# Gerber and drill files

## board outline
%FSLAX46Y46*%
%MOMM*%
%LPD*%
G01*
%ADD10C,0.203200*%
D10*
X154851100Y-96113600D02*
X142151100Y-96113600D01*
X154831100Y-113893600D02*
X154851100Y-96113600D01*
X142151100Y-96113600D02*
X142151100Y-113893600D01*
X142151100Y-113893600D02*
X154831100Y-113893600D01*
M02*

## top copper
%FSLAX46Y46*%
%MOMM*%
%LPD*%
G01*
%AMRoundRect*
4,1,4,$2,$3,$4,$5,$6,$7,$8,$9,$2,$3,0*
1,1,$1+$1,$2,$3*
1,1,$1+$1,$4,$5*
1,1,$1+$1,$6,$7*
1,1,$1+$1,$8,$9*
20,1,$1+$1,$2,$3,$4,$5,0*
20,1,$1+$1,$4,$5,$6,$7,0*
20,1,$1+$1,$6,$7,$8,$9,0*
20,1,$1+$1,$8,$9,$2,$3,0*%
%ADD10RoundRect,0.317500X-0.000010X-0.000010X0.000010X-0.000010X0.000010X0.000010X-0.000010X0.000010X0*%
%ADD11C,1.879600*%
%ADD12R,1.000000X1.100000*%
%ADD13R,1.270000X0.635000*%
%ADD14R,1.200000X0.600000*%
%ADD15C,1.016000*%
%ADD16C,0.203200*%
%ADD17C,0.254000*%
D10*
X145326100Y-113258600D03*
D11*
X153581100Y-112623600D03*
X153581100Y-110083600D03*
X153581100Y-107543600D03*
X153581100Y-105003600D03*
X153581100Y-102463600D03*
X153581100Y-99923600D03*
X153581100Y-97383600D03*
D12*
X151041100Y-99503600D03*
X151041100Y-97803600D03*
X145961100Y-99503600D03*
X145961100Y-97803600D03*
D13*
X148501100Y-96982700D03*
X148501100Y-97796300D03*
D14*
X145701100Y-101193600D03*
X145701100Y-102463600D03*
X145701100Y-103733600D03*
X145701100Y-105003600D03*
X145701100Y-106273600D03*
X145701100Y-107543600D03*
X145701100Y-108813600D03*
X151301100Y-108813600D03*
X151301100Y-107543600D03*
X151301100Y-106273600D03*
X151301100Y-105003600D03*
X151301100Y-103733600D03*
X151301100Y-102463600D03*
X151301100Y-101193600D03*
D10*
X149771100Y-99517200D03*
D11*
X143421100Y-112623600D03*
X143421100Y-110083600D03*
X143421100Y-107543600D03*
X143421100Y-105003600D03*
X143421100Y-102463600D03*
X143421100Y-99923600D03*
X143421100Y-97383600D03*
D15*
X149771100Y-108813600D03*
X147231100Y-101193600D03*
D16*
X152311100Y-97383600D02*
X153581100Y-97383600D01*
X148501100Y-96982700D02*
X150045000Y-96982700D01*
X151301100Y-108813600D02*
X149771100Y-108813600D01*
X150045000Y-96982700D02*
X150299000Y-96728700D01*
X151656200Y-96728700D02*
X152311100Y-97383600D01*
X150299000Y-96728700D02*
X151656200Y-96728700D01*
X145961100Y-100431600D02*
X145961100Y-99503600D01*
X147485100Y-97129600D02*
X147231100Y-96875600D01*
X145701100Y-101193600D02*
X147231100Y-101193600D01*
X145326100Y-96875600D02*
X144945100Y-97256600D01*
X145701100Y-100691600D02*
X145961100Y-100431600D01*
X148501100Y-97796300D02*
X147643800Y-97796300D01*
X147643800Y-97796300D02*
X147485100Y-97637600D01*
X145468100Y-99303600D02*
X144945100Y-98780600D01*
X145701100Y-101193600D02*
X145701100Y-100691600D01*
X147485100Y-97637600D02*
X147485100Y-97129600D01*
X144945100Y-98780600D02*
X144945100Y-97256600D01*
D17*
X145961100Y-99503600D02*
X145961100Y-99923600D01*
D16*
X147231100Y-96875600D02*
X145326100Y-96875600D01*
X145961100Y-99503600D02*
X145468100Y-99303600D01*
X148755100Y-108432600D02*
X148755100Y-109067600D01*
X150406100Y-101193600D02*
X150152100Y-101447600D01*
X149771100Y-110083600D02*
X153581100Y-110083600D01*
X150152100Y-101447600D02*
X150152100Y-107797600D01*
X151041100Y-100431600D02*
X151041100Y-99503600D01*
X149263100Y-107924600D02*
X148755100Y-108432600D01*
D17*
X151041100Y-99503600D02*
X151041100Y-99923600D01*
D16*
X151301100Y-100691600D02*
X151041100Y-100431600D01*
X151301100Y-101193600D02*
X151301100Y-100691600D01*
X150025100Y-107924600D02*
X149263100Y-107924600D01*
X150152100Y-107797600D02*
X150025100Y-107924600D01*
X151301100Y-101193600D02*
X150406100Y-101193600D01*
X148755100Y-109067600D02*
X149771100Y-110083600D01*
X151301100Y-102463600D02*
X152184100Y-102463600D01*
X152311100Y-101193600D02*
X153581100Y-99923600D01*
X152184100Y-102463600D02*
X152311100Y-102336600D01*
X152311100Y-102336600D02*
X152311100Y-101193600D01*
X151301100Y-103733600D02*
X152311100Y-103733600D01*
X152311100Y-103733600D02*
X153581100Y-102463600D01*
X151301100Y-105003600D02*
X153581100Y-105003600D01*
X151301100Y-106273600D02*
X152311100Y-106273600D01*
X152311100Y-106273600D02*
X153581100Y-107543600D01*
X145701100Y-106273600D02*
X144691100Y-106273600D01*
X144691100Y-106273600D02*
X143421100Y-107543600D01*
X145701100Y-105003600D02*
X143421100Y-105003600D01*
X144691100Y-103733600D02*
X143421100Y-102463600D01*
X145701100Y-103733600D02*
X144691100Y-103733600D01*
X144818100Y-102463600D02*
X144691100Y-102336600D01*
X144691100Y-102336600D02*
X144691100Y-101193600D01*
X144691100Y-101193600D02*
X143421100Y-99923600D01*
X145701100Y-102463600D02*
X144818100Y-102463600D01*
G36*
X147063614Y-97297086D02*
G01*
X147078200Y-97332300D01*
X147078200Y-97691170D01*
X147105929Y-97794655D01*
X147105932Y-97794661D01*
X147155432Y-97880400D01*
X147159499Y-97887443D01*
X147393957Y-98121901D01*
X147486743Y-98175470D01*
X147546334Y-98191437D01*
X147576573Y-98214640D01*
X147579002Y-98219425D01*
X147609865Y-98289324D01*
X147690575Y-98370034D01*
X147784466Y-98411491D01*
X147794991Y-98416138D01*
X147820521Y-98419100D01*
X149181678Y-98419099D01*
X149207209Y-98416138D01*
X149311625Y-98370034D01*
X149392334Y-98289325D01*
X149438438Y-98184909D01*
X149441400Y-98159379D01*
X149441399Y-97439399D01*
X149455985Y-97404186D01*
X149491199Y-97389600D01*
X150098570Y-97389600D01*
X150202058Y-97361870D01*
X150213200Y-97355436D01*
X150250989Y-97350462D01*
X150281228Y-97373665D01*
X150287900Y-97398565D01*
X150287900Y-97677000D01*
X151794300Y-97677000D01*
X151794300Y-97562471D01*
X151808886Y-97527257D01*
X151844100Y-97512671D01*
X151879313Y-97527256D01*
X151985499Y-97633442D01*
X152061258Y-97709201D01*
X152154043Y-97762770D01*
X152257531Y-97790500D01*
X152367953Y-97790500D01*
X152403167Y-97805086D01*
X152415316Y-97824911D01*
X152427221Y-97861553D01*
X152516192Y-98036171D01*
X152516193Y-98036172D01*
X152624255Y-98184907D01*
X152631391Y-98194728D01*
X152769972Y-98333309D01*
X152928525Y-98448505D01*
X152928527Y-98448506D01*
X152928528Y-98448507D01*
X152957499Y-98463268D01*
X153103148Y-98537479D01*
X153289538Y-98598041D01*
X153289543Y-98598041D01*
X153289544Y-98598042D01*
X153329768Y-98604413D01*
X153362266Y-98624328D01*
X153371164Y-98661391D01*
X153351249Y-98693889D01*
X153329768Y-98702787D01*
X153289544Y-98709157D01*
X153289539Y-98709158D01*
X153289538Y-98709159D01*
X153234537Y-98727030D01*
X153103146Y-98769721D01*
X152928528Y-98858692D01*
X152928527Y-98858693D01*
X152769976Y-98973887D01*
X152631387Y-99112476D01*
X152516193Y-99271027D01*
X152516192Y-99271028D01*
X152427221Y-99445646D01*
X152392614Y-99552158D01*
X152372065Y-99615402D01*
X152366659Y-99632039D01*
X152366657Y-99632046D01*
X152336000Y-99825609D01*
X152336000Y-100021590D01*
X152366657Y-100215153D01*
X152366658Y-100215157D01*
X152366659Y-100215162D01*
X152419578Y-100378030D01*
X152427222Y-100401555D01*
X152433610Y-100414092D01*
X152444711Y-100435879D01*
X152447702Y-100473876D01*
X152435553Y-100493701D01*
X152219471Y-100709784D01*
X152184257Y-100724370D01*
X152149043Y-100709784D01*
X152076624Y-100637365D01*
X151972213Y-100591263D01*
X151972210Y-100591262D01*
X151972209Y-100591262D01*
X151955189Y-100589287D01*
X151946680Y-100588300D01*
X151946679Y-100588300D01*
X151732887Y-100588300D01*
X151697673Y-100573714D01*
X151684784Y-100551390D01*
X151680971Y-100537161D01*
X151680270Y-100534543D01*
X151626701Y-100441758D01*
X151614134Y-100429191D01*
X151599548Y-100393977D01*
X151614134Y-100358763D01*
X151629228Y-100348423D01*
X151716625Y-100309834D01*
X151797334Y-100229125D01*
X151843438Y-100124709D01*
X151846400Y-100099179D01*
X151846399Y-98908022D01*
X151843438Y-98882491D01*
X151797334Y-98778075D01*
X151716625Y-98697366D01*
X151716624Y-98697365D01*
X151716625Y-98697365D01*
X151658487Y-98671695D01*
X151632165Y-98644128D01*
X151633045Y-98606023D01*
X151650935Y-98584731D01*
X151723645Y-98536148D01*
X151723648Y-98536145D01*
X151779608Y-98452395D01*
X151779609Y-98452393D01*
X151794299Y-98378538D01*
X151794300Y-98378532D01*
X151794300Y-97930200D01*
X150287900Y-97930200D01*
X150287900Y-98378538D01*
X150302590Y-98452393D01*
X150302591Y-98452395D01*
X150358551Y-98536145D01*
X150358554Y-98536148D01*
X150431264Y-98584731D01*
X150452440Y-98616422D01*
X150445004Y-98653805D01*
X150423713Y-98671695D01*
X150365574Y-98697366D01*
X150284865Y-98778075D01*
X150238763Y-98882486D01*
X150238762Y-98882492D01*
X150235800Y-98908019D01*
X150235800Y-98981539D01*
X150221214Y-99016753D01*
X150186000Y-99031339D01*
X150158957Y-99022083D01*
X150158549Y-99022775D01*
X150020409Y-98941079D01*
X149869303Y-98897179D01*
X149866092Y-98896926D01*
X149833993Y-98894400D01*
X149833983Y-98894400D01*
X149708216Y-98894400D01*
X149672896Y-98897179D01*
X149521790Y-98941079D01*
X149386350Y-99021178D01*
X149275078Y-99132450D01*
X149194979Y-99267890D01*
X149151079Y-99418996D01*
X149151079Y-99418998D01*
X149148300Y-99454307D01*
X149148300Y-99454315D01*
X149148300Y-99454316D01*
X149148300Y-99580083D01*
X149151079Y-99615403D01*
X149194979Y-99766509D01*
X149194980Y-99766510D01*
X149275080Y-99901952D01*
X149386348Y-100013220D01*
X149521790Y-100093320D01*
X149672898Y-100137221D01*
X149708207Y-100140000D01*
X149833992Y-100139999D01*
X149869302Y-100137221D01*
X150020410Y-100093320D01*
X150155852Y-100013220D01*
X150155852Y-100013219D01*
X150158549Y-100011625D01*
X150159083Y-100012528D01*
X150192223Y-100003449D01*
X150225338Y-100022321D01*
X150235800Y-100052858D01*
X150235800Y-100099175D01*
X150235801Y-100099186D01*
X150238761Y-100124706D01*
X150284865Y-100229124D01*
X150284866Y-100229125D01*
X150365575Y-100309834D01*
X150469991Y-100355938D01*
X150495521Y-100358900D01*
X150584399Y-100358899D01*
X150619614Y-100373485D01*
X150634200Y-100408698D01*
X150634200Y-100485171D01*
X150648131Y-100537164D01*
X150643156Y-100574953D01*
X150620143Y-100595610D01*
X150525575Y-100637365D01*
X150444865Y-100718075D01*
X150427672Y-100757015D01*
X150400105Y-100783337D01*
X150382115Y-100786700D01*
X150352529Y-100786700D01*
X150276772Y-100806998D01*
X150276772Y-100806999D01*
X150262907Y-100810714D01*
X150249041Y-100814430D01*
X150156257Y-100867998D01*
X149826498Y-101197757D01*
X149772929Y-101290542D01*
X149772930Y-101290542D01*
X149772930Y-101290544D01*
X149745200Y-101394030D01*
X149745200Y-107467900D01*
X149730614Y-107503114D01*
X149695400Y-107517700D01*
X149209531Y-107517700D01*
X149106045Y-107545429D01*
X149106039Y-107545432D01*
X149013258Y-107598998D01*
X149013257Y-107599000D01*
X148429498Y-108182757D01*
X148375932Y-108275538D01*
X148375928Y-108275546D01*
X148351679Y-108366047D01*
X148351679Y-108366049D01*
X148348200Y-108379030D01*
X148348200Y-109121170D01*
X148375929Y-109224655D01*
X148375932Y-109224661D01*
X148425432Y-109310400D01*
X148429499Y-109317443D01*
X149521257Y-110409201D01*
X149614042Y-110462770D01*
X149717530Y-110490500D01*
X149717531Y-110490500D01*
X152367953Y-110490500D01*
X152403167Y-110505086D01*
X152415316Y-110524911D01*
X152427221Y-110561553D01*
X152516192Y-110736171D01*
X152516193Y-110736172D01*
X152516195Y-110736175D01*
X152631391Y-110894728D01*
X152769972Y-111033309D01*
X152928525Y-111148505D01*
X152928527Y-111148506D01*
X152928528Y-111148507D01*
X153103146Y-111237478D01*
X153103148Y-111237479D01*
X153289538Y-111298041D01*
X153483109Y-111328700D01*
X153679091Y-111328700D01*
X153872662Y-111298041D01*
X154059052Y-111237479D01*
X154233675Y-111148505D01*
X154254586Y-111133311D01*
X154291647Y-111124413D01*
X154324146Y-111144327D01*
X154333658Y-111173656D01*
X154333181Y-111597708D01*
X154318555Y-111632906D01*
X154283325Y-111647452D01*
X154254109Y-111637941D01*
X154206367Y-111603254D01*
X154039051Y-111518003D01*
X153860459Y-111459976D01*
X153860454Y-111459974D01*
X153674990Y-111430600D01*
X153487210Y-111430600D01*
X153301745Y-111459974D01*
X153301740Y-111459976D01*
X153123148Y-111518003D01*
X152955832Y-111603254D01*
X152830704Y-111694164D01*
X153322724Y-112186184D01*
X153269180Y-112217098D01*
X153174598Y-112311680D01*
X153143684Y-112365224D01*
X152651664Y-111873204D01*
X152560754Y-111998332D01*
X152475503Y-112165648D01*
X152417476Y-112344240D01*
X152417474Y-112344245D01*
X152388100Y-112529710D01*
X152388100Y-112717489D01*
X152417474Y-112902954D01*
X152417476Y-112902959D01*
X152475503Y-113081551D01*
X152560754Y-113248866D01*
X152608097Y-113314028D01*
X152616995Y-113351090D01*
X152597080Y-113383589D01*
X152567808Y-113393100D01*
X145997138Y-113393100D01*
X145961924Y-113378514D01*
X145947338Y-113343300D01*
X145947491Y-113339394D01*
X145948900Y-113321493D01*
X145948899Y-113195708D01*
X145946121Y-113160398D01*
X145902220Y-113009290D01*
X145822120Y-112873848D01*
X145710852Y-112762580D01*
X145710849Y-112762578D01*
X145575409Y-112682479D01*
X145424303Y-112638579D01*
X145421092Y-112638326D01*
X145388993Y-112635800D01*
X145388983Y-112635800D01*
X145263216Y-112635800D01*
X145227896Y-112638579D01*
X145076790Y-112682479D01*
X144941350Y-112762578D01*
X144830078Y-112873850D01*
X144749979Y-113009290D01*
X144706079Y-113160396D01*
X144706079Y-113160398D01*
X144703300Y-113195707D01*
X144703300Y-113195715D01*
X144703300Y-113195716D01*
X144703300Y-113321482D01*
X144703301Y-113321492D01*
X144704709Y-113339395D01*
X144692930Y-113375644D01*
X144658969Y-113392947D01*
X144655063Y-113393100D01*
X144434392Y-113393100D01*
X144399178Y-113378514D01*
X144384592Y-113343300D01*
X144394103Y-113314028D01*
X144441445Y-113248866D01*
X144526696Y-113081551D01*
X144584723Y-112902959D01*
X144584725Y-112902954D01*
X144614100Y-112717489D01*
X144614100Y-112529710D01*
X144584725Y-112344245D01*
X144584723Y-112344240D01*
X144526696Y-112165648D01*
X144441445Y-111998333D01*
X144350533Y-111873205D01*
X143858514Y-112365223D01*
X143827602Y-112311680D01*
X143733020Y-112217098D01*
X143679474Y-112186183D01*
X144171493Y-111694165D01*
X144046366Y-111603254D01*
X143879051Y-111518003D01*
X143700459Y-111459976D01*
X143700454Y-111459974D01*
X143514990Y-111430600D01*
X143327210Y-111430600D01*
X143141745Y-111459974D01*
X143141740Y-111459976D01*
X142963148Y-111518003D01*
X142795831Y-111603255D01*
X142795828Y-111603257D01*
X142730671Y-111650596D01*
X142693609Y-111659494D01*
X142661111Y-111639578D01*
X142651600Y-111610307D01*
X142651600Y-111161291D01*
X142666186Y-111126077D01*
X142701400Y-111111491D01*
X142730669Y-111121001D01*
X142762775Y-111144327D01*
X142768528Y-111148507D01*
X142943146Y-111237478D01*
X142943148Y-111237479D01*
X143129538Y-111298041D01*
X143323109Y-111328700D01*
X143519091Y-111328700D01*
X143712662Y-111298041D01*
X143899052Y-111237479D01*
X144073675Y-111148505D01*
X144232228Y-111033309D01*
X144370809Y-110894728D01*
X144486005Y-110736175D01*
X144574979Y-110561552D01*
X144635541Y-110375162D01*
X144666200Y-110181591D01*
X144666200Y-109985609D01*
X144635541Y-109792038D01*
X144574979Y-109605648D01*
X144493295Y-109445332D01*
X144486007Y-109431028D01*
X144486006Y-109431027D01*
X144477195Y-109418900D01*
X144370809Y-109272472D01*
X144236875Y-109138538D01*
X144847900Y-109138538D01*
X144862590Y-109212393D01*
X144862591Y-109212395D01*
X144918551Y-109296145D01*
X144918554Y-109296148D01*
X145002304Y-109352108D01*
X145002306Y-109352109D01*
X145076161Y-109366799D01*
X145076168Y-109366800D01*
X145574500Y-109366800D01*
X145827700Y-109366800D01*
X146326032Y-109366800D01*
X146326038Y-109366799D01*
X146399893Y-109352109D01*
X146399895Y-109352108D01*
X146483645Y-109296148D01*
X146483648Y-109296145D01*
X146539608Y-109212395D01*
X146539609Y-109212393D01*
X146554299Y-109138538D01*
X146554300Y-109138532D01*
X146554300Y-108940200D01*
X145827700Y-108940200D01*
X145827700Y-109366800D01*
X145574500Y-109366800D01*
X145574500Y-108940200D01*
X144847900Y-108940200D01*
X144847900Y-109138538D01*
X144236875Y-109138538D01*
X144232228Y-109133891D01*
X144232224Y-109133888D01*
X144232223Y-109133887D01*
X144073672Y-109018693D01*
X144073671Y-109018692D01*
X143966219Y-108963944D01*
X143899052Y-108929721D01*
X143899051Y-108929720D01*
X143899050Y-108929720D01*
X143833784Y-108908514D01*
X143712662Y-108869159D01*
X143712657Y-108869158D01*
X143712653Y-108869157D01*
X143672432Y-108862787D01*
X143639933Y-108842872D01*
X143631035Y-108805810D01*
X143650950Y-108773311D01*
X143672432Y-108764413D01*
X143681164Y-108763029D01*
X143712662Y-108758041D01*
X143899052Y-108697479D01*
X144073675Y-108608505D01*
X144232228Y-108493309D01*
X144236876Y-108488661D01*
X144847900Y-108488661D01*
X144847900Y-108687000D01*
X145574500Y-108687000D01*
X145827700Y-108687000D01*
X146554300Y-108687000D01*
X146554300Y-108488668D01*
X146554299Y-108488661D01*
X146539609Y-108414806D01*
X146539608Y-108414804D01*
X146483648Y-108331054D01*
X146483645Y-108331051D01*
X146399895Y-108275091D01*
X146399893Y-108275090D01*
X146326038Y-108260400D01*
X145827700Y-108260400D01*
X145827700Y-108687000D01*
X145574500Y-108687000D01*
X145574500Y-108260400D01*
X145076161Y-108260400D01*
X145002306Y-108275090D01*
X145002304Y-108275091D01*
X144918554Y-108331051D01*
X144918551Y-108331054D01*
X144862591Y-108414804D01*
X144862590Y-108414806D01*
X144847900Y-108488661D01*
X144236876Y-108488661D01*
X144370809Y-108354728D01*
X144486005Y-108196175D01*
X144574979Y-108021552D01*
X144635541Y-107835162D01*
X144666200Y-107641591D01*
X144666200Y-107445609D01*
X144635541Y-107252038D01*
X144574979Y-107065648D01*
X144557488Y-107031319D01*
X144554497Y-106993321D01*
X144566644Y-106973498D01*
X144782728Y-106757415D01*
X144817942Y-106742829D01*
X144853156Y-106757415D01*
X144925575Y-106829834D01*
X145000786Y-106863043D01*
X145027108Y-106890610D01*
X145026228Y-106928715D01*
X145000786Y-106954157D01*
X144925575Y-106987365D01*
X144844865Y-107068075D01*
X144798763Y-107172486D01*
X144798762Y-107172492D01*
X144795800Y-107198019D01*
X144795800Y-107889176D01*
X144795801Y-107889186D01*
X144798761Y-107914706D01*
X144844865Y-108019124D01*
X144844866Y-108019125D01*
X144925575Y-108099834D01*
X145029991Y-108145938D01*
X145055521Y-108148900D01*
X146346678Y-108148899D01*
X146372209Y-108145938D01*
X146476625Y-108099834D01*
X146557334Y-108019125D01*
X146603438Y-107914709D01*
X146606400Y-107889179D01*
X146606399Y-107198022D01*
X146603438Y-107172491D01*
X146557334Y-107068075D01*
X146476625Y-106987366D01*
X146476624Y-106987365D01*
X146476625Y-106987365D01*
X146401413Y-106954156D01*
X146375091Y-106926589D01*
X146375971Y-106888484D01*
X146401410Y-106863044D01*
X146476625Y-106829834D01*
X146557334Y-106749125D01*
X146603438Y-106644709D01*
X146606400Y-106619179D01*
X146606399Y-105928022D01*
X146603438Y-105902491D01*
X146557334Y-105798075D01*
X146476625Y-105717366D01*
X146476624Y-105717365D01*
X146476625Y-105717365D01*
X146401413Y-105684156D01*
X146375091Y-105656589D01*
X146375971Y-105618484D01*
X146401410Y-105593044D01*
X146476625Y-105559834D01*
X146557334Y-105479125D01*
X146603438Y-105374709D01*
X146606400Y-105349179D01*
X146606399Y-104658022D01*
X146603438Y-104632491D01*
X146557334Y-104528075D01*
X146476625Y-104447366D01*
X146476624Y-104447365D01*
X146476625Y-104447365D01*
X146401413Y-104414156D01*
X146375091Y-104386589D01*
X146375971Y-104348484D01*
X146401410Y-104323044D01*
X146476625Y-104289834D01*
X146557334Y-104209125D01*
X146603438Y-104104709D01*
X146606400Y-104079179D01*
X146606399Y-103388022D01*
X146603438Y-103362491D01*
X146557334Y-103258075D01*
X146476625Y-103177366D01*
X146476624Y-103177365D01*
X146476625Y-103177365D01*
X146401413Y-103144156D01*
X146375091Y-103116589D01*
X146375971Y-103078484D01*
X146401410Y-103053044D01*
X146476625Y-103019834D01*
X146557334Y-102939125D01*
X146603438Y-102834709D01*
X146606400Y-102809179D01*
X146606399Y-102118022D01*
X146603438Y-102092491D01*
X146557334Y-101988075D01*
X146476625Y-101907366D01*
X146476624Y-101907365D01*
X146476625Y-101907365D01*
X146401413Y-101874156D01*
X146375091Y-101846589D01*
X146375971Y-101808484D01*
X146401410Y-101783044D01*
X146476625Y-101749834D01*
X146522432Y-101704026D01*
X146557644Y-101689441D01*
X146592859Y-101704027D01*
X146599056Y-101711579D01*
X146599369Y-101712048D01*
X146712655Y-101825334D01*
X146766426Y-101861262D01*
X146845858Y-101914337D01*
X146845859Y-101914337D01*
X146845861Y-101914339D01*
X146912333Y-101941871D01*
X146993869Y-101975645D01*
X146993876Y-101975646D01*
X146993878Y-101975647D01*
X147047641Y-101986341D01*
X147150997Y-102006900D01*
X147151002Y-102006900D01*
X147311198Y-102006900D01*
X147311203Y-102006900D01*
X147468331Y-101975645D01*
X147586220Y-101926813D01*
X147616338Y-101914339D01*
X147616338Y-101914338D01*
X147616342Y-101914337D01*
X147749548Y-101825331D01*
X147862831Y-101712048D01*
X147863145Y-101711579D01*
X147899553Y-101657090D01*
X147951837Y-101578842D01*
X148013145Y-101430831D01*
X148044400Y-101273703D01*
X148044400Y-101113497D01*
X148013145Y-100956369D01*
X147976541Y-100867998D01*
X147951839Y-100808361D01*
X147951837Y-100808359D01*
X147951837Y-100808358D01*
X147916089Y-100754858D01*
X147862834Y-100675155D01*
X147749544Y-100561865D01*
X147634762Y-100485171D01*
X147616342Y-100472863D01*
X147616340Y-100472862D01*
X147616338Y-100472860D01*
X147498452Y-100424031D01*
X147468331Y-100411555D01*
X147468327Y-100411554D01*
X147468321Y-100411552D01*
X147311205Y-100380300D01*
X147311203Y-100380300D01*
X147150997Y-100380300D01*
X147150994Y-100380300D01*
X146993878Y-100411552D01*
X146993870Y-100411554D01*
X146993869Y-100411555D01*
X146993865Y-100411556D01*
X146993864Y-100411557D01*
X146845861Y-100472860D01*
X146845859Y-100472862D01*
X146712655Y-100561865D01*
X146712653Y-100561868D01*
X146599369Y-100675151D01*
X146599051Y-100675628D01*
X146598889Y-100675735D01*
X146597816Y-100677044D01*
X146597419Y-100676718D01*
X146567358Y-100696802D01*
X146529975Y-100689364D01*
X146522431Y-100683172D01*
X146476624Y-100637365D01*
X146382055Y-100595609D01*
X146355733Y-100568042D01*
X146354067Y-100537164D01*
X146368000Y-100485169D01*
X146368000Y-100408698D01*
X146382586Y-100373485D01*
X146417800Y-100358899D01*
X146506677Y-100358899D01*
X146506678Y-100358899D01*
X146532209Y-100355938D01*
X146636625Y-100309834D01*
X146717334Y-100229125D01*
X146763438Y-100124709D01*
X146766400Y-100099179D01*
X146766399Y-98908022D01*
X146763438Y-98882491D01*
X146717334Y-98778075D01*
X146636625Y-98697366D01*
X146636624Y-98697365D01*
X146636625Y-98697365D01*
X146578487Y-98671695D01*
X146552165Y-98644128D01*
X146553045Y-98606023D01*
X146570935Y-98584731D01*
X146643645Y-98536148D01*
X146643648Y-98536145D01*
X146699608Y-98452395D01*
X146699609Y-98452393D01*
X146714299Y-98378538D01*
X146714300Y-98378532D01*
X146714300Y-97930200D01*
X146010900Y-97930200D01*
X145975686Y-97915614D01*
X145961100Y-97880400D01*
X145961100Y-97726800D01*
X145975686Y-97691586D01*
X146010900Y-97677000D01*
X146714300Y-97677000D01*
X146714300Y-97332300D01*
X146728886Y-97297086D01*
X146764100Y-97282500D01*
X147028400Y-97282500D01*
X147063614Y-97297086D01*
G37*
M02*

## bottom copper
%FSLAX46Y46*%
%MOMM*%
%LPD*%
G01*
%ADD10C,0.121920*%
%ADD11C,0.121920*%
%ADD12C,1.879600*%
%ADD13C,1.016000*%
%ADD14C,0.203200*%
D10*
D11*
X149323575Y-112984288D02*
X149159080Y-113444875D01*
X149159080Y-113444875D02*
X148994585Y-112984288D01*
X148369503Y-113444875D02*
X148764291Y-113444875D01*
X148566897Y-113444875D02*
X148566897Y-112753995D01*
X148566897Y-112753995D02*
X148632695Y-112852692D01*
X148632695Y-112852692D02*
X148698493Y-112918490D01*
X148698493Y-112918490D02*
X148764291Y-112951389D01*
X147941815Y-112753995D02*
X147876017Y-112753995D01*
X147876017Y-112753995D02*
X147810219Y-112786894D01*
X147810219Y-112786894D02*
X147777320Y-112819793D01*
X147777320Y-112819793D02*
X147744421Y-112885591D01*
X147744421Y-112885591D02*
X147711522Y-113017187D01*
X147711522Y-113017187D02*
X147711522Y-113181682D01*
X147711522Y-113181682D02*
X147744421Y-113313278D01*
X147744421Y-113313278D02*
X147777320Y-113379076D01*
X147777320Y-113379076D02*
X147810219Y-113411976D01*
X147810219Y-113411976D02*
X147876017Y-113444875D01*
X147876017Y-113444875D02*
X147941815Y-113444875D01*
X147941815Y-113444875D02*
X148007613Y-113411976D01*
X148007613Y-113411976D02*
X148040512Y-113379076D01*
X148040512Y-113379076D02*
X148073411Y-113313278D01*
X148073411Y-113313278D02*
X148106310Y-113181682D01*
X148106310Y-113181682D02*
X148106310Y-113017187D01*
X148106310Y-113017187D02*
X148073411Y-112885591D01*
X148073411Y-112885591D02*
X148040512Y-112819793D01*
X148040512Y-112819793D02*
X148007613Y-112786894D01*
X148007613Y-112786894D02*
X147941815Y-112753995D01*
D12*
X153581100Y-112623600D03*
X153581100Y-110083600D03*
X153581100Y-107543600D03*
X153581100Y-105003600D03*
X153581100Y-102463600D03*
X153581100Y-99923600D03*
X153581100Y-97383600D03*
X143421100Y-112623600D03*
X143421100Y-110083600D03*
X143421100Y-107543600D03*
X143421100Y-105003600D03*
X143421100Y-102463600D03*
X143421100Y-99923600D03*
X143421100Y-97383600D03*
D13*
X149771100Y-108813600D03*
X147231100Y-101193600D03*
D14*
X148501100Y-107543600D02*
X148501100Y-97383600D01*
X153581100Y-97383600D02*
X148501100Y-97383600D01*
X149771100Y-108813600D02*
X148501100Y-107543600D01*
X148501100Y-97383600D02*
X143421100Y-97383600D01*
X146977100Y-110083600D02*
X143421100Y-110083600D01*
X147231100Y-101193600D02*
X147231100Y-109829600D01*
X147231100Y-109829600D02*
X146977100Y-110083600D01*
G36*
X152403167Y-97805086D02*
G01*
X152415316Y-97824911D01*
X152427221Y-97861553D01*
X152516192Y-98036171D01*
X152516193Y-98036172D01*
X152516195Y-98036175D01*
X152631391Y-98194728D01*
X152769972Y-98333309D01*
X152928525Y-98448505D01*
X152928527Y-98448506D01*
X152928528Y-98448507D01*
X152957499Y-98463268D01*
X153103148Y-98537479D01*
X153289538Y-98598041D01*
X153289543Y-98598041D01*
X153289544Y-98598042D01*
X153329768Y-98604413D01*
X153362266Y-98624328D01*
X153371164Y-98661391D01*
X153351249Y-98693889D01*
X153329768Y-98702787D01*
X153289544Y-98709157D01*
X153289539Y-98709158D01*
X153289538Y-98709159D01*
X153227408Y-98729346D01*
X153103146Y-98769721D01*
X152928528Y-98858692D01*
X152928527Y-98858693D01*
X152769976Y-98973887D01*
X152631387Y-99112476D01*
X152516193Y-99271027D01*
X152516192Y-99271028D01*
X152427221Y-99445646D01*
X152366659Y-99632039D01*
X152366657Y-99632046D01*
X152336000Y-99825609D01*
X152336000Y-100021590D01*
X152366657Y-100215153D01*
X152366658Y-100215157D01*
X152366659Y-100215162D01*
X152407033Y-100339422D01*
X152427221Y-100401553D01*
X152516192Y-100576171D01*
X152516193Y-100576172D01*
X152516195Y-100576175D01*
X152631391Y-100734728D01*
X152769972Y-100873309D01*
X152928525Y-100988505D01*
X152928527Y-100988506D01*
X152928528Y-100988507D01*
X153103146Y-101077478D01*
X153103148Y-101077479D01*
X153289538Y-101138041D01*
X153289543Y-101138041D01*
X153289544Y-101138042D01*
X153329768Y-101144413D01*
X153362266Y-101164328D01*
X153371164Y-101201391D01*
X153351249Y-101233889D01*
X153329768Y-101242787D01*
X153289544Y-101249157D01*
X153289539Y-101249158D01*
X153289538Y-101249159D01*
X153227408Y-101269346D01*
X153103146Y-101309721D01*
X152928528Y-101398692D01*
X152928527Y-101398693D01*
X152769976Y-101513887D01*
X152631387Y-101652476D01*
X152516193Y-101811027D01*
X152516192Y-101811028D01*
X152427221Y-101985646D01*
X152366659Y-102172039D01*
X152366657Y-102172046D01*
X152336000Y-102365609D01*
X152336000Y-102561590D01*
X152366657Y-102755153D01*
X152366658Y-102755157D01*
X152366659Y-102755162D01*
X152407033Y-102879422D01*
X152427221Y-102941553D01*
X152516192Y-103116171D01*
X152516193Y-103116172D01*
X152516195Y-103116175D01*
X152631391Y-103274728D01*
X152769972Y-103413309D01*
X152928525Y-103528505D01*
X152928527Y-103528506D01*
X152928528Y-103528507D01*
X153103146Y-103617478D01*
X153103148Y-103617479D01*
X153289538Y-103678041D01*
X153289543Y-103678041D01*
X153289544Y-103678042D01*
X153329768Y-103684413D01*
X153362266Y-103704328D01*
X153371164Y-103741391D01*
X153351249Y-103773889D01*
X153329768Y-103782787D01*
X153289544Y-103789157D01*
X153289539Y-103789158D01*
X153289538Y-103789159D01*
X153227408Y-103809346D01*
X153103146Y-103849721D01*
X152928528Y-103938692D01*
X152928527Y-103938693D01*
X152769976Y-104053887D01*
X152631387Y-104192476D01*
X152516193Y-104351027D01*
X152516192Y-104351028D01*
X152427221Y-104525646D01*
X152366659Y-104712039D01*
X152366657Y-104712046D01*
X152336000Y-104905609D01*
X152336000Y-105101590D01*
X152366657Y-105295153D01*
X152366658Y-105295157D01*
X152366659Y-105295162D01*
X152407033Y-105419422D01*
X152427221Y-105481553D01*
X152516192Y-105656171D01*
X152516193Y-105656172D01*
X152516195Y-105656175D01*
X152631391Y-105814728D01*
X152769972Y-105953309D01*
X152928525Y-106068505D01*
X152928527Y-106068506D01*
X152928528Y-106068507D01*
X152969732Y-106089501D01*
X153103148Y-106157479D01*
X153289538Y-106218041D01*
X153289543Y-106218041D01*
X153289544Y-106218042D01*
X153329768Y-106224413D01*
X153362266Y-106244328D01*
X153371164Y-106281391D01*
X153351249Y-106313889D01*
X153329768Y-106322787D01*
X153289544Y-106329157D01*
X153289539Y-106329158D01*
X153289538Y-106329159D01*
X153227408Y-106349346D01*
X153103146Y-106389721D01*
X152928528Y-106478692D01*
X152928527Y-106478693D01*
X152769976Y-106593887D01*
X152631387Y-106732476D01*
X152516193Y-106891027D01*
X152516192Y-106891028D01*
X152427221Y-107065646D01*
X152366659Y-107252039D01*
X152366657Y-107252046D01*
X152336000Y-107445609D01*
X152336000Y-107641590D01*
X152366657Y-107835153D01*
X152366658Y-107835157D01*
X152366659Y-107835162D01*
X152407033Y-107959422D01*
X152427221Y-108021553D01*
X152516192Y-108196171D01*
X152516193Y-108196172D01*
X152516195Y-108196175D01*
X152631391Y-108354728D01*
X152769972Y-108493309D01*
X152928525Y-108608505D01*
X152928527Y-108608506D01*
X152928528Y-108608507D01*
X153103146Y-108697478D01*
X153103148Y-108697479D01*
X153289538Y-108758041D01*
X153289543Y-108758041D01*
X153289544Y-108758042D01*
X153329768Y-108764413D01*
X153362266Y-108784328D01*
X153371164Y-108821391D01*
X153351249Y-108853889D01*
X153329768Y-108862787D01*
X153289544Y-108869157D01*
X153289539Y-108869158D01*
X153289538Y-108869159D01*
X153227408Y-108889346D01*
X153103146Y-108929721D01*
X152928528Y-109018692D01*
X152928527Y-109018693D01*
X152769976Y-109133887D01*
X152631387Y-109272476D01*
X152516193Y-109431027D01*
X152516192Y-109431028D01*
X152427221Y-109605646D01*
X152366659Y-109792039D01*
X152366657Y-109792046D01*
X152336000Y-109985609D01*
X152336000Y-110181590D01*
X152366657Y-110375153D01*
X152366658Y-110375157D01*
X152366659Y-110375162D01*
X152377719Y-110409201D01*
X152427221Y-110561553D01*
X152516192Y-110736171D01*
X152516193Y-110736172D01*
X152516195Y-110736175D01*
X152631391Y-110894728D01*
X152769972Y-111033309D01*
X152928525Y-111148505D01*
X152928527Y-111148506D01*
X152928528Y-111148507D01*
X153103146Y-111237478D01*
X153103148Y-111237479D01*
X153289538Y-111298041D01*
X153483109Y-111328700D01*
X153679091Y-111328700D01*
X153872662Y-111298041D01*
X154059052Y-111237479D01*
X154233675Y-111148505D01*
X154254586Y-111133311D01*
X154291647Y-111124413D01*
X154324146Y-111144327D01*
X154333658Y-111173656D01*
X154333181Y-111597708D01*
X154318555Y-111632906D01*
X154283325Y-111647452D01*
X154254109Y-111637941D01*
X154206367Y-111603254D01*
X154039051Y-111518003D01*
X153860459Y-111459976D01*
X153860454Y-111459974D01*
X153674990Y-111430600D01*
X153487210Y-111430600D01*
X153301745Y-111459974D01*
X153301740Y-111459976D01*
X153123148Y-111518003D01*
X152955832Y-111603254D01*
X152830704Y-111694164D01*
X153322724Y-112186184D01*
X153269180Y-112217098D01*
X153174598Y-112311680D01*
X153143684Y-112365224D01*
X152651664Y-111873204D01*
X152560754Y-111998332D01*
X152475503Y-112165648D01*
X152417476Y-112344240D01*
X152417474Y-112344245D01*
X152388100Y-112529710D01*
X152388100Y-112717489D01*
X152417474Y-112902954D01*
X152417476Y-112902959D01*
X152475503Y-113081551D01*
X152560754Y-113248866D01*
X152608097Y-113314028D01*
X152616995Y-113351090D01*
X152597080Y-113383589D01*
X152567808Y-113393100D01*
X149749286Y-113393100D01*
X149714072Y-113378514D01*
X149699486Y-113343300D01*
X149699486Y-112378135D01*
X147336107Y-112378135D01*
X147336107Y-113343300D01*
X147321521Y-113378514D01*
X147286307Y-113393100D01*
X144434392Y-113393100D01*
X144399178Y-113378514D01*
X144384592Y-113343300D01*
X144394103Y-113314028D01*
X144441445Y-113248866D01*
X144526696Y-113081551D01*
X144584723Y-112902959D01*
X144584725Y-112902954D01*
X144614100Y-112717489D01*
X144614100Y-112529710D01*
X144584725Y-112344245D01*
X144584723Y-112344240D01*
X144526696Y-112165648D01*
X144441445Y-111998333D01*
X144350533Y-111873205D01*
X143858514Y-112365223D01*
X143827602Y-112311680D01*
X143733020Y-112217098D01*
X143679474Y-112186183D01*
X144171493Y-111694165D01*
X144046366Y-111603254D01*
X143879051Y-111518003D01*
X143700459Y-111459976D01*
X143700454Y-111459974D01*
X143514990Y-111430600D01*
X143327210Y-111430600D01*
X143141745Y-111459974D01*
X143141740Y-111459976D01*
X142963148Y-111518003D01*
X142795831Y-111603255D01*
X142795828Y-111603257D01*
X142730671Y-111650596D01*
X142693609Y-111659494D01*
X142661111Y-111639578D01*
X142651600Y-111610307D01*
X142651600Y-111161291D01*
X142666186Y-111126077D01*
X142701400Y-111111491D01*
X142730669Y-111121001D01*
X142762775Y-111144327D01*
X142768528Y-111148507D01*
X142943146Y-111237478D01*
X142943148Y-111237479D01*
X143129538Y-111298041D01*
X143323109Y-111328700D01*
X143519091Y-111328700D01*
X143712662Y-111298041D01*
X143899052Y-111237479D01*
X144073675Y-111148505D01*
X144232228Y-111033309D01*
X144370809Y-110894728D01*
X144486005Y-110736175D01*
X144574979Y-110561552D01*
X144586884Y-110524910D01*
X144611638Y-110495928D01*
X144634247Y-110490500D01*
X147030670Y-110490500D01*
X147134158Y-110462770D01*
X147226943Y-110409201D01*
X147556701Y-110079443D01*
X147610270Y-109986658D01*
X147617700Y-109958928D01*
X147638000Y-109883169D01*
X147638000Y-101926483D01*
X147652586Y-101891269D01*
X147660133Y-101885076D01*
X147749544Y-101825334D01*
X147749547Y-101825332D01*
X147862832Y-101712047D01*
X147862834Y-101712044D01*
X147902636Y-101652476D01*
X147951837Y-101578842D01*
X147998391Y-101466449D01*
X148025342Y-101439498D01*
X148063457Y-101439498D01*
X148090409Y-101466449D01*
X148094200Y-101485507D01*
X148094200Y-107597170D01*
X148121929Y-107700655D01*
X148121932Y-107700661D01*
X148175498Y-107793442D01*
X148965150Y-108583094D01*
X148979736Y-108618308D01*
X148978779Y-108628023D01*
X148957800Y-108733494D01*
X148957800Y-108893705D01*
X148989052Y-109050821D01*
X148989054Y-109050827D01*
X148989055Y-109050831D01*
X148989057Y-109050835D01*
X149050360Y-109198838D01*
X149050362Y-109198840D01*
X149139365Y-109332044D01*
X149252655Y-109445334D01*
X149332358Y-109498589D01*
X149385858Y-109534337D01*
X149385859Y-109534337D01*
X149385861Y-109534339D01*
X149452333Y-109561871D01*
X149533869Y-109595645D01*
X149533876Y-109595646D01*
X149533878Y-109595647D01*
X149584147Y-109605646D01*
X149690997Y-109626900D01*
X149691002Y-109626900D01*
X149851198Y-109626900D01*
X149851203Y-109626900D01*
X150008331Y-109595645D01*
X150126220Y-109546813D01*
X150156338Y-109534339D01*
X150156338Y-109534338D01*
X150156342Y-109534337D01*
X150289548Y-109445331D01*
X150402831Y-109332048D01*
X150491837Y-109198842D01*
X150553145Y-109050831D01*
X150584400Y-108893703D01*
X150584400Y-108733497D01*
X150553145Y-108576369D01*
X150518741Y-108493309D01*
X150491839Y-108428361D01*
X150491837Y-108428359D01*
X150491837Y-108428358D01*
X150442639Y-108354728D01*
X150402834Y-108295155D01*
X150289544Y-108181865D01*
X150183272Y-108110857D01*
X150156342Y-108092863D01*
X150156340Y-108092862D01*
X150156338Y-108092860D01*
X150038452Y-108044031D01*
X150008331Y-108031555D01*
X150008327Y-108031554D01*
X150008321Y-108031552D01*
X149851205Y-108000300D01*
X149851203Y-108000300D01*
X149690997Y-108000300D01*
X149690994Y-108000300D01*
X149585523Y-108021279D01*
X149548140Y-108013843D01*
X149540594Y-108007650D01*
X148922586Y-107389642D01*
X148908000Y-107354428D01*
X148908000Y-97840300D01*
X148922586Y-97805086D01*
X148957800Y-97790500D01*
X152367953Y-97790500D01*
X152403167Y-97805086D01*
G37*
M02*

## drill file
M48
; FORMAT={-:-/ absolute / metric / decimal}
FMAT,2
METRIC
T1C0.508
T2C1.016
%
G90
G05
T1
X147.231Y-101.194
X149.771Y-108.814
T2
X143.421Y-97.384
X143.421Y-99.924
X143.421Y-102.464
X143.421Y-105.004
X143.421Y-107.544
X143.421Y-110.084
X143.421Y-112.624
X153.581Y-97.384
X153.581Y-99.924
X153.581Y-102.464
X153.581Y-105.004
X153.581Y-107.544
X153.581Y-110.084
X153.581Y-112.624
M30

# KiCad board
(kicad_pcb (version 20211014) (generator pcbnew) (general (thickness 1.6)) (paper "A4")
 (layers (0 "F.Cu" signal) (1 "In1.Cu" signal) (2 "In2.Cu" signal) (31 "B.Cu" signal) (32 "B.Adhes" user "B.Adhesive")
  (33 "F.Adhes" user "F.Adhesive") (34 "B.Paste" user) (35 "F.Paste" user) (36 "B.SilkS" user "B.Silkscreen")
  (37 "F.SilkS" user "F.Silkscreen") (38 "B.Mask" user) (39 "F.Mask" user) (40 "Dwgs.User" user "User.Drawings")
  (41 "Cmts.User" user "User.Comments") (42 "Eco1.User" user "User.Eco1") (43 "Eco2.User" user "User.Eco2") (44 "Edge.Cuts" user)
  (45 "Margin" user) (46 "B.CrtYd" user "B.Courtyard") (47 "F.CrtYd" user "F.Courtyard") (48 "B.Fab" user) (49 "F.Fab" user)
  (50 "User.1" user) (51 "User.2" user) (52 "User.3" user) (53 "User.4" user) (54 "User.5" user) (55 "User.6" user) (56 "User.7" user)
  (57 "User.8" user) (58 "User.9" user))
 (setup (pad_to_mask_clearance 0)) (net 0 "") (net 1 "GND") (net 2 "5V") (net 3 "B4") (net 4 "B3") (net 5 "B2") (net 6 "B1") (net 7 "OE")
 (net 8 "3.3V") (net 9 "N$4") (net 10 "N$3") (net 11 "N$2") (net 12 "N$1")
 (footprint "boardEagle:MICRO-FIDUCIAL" (layer "F.Cu") (at 145.3261 113.2586)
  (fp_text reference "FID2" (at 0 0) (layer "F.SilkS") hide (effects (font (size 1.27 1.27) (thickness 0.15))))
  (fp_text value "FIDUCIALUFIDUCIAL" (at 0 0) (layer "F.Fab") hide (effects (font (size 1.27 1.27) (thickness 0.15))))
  (pad "1" smd roundrect (at 0 0) (size 0.635 0.635) (layers "F.Cu" "F.Mask") (roundrect_rratio 0.5) (solder_mask_margin 0.1016)))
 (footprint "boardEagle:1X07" (layer "F.Cu") (at 153.5811 112.6236 90)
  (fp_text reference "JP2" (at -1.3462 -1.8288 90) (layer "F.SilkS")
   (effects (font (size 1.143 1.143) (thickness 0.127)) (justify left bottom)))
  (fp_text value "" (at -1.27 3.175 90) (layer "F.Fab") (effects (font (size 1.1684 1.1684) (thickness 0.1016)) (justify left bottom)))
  (pad "1" thru_hole circle (at 0 0 180) (size 1.8796 1.8796) (drill 1.016) (layers *.Cu *.Mask) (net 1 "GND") (solder_mask_margin 0.1016))
  (pad "2" thru_hole circle (at 2.54 0 180) (size 1.8796 1.8796) (drill 1.016) (layers *.Cu *.Mask) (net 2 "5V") (solder_mask_margin 0.1016))
  (pad "3" thru_hole circle (at 5.08 0 180) (size 1.8796 1.8796) (drill 1.016) (layers *.Cu *.Mask) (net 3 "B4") (solder_mask_margin 0.1016))
  (pad "4" thru_hole circle (at 7.62 0 180) (size 1.8796 1.8796) (drill 1.016) (layers *.Cu *.Mask) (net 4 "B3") (solder_mask_margin 0.1016))
  (pad "5" thru_hole circle (at 10.16 0 180) (size 1.8796 1.8796) (drill 1.016) (layers *.Cu *.Mask) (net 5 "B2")
   (solder_mask_margin 0.1016))
  (pad "6" thru_hole circle (at 12.7 0 180) (size 1.8796 1.8796) (drill 1.016) (layers *.Cu *.Mask) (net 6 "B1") (solder_mask_margin 0.1016))
  (pad "7" thru_hole circle (at 15.24 0 180) (size 1.8796 1.8796) (drill 1.016) (layers *.Cu *.Mask) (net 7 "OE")
   (solder_mask_margin 0.1016)))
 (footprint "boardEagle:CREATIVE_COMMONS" (layer "F.Cu") (at 64.6811 112.6236)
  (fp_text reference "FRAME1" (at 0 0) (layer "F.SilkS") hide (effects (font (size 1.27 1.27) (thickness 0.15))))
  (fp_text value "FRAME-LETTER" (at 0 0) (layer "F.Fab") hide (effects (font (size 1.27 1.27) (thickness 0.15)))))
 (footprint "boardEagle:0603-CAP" (layer "F.Cu") (at 151.0411 98.6536 90)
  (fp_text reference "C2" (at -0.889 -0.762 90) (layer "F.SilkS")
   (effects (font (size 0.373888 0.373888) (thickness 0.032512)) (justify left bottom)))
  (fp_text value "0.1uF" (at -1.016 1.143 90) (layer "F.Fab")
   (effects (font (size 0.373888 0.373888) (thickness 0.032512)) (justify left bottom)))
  (pad "1" smd rect (at -0.85 0 90) (size 1.1 1) (layers "F.Cu" "F.Paste" "F.Mask") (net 2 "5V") (solder_mask_margin 0.1016))
  (pad "2" smd rect (at 0.85 0 90) (size 1.1 1) (layers "F.Cu" "F.Paste" "F.Mask") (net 1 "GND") (solder_mask_margin 0.1016)))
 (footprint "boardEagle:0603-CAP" (layer "F.Cu") (at 145.9611 98.6536 90)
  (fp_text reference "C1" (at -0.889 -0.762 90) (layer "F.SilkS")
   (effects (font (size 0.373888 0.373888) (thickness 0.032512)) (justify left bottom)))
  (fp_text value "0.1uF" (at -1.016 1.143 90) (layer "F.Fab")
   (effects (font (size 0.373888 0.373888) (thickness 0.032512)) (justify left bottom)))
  (pad "1" smd rect (at -0.85 0 90) (size 1.1 1) (layers "F.Cu" "F.Paste" "F.Mask") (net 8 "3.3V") (solder_mask_margin 0.1016))
  (pad "2" smd rect (at 0.85 0 90) (size 1.1 1) (layers "F.Cu" "F.Paste" "F.Mask") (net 1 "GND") (solder_mask_margin 0.1016)))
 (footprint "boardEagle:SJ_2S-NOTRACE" (layer "F.Cu") (at 148.5011 97.3836 -90)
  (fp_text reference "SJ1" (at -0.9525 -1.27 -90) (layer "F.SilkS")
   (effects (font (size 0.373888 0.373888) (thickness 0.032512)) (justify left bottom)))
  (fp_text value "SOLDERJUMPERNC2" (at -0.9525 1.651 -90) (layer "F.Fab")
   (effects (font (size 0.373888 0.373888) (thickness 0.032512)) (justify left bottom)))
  (pad "1" smd rect (at -0.4009 0 90) (size 0.635 1.27) (layers "F.Cu" "F.Mask") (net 7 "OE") (solder_mask_margin 0.1016))
  (pad "2" smd rect (at 0.4127 0 270) (size 0.635 1.27) (layers "F.Cu" "F.Mask") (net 8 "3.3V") (solder_mask_margin 0.1016)))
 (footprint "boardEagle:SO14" (layer "F.Cu") (at 148.5011 105.0036 -90)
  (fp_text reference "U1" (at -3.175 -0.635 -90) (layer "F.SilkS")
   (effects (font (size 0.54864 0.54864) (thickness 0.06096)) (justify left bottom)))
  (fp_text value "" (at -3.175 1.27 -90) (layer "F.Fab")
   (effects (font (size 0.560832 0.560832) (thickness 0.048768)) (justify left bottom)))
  (pad "1" smd rect (at -3.81 2.8 270) (size 0.6 1.2) (layers "F.Cu" "F.Paste" "F.Mask") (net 8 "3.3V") (solder_mask_margin 0.1016))
  (pad "2" smd rect (at -2.54 2.8 270) (size 0.6 1.2) (layers "F.Cu" "F.Paste" "F.Mask") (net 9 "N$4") (solder_mask_margin 0.1016))
  (pad "3" smd rect (at -1.27 2.8 270) (size 0.6 1.2) (layers "F.Cu" "F.Paste" "F.Mask") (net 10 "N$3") (solder_mask_margin 0.1016))
  (pad "4" smd rect (at 0 2.8 270) (size 0.6 1.2) (layers "F.Cu" "F.Paste" "F.Mask") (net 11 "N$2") (solder_mask_margin 0.1016))
  (pad "5" smd rect (at 1.27 2.8 270) (size 0.6 1.2) (layers "F.Cu" "F.Paste" "F.Mask") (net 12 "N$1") (solder_mask_margin 0.1016))
  (pad "6" smd rect (at 2.54 2.8 270) (size 0.6 1.2) (layers "F.Cu" "F.Paste" "F.Mask") (solder_mask_margin 0.1016))
  (pad "7" smd rect (at 3.81 2.8 270) (size 0.6 1.2) (layers "F.Cu" "F.Paste" "F.Mask") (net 1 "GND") (solder_mask_margin 0.1016))
  (pad "8" smd rect (at 3.81 -2.8 270) (size 0.6 1.2) (layers "F.Cu" "F.Paste" "F.Mask") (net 7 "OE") (solder_mask_margin 0.1016))
  (pad "9" smd rect (at 2.54 -2.8 270) (size 0.6 1.2) (layers "F.Cu" "F.Paste" "F.Mask") (solder_mask_margin 0.1016))
  (pad "10" smd rect (at 1.27 -2.8 270) (size 0.6 1.2) (layers "F.Cu" "F.Paste" "F.Mask") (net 3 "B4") (solder_mask_margin 0.1016))
  (pad "11" smd rect (at 0 -2.8 270) (size 0.6 1.2) (layers "F.Cu" "F.Paste" "F.Mask") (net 4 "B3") (solder_mask_margin 0.1016))
  (pad "12" smd rect (at -1.27 -2.8 270) (size 0.6 1.2) (layers "F.Cu" "F.Paste" "F.Mask") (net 5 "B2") (solder_mask_margin 0.1016))
  (pad "13" smd rect (at -2.54 -2.8 270) (size 0.6 1.2) (layers "F.Cu" "F.Paste" "F.Mask") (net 6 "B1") (solder_mask_margin 0.1016))
  (pad "14" smd rect (at -3.81 -2.8 270) (size 0.6 1.2) (layers "F.Cu" "F.Paste" "F.Mask") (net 2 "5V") (solder_mask_margin 0.1016)))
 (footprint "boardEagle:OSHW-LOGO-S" (layer "F.Cu") (at 146.5961 111.6076)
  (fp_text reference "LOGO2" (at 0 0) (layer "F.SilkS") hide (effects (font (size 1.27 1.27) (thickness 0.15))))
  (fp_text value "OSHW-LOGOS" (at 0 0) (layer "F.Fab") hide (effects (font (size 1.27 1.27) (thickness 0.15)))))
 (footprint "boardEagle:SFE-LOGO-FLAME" (layer "F.Cu") (at 150.1521 113.0046)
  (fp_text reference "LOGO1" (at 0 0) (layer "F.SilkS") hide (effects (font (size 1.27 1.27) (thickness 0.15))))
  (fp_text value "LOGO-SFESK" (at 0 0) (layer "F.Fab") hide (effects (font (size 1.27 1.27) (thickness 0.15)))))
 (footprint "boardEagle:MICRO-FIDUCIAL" (layer "F.Cu") (at 149.7711 99.5172)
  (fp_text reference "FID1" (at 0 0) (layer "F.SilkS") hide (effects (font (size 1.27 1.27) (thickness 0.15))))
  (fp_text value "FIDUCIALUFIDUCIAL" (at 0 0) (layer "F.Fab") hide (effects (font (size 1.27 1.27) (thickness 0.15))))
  (pad "1" smd roundrect (at 0 0) (size 0.635 0.635) (layers "F.Cu" "F.Mask") (roundrect_rratio 0.5) (solder_mask_margin 0.1016)))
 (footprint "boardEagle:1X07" (layer "F.Cu") (at 143.4211 112.6236 90)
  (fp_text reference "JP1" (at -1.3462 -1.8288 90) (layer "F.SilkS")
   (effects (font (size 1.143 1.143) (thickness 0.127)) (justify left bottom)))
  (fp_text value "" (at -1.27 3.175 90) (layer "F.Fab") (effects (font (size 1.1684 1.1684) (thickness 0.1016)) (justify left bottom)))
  (pad "1" thru_hole circle (at 0 0 180) (size 1.8796 1.8796) (drill 1.016) (layers *.Cu *.Mask) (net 1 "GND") (solder_mask_margin 0.1016))
  (pad "2" thru_hole circle (at 2.54 0 180) (size 1.8796 1.8796) (drill 1.016) (layers *.Cu *.Mask) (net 8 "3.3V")
   (solder_mask_margin 0.1016))
  (pad "3" thru_hole circle (at 5.08 0 180) (size 1.8796 1.8796) (drill 1.016) (layers *.Cu *.Mask) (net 12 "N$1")
   (solder_mask_margin 0.1016))
  (pad "4" thru_hole circle (at 7.62 0 180) (size 1.8796 1.8796) (drill 1.016) (layers *.Cu *.Mask) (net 11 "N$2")
   (solder_mask_margin 0.1016))
  (pad "5" thru_hole circle (at 10.16 0 180) (size 1.8796 1.8796) (drill 1.016) (layers *.Cu *.Mask) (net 10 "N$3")
   (solder_mask_margin 0.1016))
  (pad "6" thru_hole circle (at 12.7 0 180) (size 1.8796 1.8796) (drill 1.016) (layers *.Cu *.Mask) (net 9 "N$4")
   (solder_mask_margin 0.1016))
  (pad "7" thru_hole circle (at 15.24 0 180) (size 1.8796 1.8796) (drill 1.016) (layers *.Cu *.Mask) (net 7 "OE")
   (solder_mask_margin 0.1016)))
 (gr_line (start 154.8511 96.1136) (end 142.1511 96.1136) (layer "Edge.Cuts") (width 0.2032))
 (gr_line (start 154.8311 113.8936) (end 154.8511 96.1136) (layer "Edge.Cuts") (width 0.2032))
 (gr_line (start 142.1511 96.1136) (end 142.1511 113.8936) (layer "Edge.Cuts") (width 0.2032))
 (gr_line (start 142.1511 113.8936) (end 154.8311 113.8936) (layer "Edge.Cuts") (width 0.2032))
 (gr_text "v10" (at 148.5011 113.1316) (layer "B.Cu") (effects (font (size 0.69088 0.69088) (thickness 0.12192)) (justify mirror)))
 (segment (start 152.3111 97.3836) (end 153.5811 97.3836) (width 0.2032) (layer "F.Cu") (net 7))
 (segment (start 148.5011 96.9827) (end 150.045 96.9827) (width 0.2032) (layer "F.Cu") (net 7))
 (segment (start 151.3011 108.8136) (end 149.7711 108.8136) (width 0.2032) (layer "F.Cu") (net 7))
 (segment (start 150.045 96.9827) (end 150.299 96.7287) (width 0.2032) (layer "F.Cu") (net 7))
 (segment (start 151.6562 96.7287) (end 152.3111 97.3836) (width 0.2032) (layer "F.Cu") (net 7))
 (segment (start 150.299 96.7287) (end 151.6562 96.7287) (width 0.2032) (layer "F.Cu") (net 7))
 (via (at 149.7711 108.8136) (size 1.016) (drill 0.508) (layers "F.Cu" "B.Cu") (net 7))
 (segment (start 148.5011 107.5436) (end 148.5011 97.3836) (width 0.2032) (layer "B.Cu") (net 7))
 (segment (start 153.5811 97.3836) (end 148.5011 97.3836) (width 0.2032) (layer "B.Cu") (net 7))
 (segment (start 149.7711 108.8136) (end 148.5011 107.5436) (width 0.2032) (layer "B.Cu") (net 7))
 (segment (start 148.5011 97.3836) (end 143.4211 97.3836) (width 0.2032) (layer "B.Cu") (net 7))
 (segment (start 145.9611 100.4316) (end 145.9611 99.5036) (width 0.2032) (layer "F.Cu") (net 8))
 (segment (start 147.4851 97.1296) (end 147.2311 96.8756) (width 0.2032) (layer "F.Cu") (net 8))
 (segment (start 145.7011 101.1936) (end 147.2311 101.1936) (width 0.2032) (layer "F.Cu") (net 8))
 (segment (start 145.3261 96.8756) (end 144.9451 97.2566) (width 0.2032) (layer "F.Cu") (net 8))
 (segment (start 145.7011 100.6916) (end 145.9611 100.4316) (width 0.2032) (layer "F.Cu") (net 8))
 (segment (start 148.5011 97.7963) (end 147.6438 97.7963) (width 0.2032) (layer "F.Cu") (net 8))
 (segment (start 147.6438 97.7963) (end 147.4851 97.6376) (width 0.2032) (layer "F.Cu") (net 8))
 (segment (start 145.4681 99.3036) (end 144.9451 98.7806) (width 0.2032) (layer "F.Cu") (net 8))
 (segment (start 145.7011 101.1936) (end 145.7011 100.6916) (width 0.2032) (layer "F.Cu") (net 8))
 (segment (start 147.4851 97.6376) (end 147.4851 97.1296) (width 0.2032) (layer "F.Cu") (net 8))
 (segment (start 144.9451 98.7806) (end 144.9451 97.2566) (width 0.2032) (layer "F.Cu") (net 8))
 (segment (start 145.9611 99.5036) (end 145.9611 99.9236) (width 0.254) (layer "F.Cu") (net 8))
 (segment (start 147.2311 96.8756) (end 145.3261 96.8756) (width 0.2032) (layer "F.Cu") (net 8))
 (segment (start 145.9611 99.5036) (end 145.4681 99.3036) (width 0.2032) (layer "F.Cu") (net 8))
 (via (at 147.2311 101.1936) (size 1.016) (drill 0.508) (layers "F.Cu" "B.Cu") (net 8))
 (segment (start 146.9771 110.0836) (end 143.4211 110.0836) (width 0.2032) (layer "B.Cu") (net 8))
 (segment (start 147.2311 101.1936) (end 147.2311 109.8296) (width 0.2032) (layer "B.Cu") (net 8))
 (segment (start 147.2311 109.8296) (end 146.9771 110.0836) (width 0.2032) (layer "B.Cu") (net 8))
 (segment (start 148.7551 108.4326) (end 148.7551 109.0676) (width 0.2032) (layer "F.Cu") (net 2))
 (segment (start 150.4061 101.1936) (end 150.1521 101.4476) (width 0.2032) (layer "F.Cu") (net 2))
 (segment (start 149.7711 110.0836) (end 153.5811 110.0836) (width 0.2032) (layer "F.Cu") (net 2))
 (segment (start 150.1521 101.4476) (end 150.1521 107.7976) (width 0.2032) (layer "F.Cu") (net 2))
 (segment (start 151.0411 100.4316) (end 151.0411 99.5036) (width 0.2032) (layer "F.Cu") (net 2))
 (segment (start 149.2631 107.9246) (end 148.7551 108.4326) (width 0.2032) (layer "F.Cu") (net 2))
 (segment (start 151.0411 99.5036) (end 151.0411 99.9236) (width 0.254) (layer "F.Cu") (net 2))
 (segment (start 151.3011 100.6916) (end 151.0411 100.4316) (width 0.2032) (layer "F.Cu") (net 2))
 (segment (start 151.3011 101.1936) (end 151.3011 100.6916) (width 0.2032) (layer "F.Cu") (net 2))
 (segment (start 150.0251 107.9246) (end 149.2631 107.9246) (width 0.2032) (layer "F.Cu") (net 2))
 (segment (start 150.1521 107.7976) (end 150.0251 107.9246) (width 0.2032) (layer "F.Cu") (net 2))
 (segment (start 151.3011 101.1936) (end 150.4061 101.1936) (width 0.2032) (layer "F.Cu") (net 2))
 (segment (start 148.7551 109.0676) (end 149.7711 110.0836) (width 0.2032) (layer "F.Cu") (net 2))
 (segment (start 151.3011 102.4636) (end 152.1841 102.4636) (width 0.2032) (layer "F.Cu") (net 6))
 (segment (start 152.3111 101.1936) (end 153.5811 99.9236) (width 0.2032) (layer "F.Cu") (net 6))
 (segment (start 152.1841 102.4636) (end 152.3111 102.3366) (width 0.2032) (layer "F.Cu") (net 6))
 (segment (start 152.3111 102.3366) (end 152.3111 101.1936) (width 0.2032) (layer "F.Cu") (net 6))
 (segment (start 151.3011 103.7336) (end 152.3111 103.7336) (width 0.2032) (layer "F.Cu") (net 5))
 (segment (start 152.3111 103.7336) (end 153.5811 102.4636) (width 0.2032) (layer "F.Cu") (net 5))
 (segment (start 151.3011 105.0036) (end 153.5811 105.0036) (width 0.2032) (layer "F.Cu") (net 4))
 (segment (start 151.3011 106.2736) (end 152.3111 106.2736) (width 0.2032) (layer "F.Cu") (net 3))
 (segment (start 152.3111 106.2736) (end 153.5811 107.5436) (width 0.2032) (layer "F.Cu") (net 3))
 (segment (start 145.7011 106.2736) (end 144.6911 106.2736) (width 0.2032) (layer "F.Cu") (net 12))
 (segment (start 144.6911 106.2736) (end 143.4211 107.5436) (width 0.2032) (layer "F.Cu") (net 12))
 (segment (start 145.7011 105.0036) (end 143.4211 105.0036) (width 0.2032) (layer "F.Cu") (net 11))
 (segment (start 144.6911 103.7336) (end 143.4211 102.4636) (width 0.2032) (layer "F.Cu") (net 10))
 (segment (start 145.7011 103.7336) (end 144.6911 103.7336) (width 0.2032) (layer "F.Cu") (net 10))
 (segment (start 144.8181 102.4636) (end 144.6911 102.3366) (width 0.2032) (layer "F.Cu") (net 9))
 (segment (start 144.6911 102.3366) (end 144.6911 101.1936) (width 0.2032) (layer "F.Cu") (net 9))
 (segment (start 144.6911 101.1936) (end 143.4211 99.9236) (width 0.2032) (layer "F.Cu") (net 9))
 (segment (start 145.7011 102.4636) (end 144.8181 102.4636) (width 0.2032) (layer "F.Cu") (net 9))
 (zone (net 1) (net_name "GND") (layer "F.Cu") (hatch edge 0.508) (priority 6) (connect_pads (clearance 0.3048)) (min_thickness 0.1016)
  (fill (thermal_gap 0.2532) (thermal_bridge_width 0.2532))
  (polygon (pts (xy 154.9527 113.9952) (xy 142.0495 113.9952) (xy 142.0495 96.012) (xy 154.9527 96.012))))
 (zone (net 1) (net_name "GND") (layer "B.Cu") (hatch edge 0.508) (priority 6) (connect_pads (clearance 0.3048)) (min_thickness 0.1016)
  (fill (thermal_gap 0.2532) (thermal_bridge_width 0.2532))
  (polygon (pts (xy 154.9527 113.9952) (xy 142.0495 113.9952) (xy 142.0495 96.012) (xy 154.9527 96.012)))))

